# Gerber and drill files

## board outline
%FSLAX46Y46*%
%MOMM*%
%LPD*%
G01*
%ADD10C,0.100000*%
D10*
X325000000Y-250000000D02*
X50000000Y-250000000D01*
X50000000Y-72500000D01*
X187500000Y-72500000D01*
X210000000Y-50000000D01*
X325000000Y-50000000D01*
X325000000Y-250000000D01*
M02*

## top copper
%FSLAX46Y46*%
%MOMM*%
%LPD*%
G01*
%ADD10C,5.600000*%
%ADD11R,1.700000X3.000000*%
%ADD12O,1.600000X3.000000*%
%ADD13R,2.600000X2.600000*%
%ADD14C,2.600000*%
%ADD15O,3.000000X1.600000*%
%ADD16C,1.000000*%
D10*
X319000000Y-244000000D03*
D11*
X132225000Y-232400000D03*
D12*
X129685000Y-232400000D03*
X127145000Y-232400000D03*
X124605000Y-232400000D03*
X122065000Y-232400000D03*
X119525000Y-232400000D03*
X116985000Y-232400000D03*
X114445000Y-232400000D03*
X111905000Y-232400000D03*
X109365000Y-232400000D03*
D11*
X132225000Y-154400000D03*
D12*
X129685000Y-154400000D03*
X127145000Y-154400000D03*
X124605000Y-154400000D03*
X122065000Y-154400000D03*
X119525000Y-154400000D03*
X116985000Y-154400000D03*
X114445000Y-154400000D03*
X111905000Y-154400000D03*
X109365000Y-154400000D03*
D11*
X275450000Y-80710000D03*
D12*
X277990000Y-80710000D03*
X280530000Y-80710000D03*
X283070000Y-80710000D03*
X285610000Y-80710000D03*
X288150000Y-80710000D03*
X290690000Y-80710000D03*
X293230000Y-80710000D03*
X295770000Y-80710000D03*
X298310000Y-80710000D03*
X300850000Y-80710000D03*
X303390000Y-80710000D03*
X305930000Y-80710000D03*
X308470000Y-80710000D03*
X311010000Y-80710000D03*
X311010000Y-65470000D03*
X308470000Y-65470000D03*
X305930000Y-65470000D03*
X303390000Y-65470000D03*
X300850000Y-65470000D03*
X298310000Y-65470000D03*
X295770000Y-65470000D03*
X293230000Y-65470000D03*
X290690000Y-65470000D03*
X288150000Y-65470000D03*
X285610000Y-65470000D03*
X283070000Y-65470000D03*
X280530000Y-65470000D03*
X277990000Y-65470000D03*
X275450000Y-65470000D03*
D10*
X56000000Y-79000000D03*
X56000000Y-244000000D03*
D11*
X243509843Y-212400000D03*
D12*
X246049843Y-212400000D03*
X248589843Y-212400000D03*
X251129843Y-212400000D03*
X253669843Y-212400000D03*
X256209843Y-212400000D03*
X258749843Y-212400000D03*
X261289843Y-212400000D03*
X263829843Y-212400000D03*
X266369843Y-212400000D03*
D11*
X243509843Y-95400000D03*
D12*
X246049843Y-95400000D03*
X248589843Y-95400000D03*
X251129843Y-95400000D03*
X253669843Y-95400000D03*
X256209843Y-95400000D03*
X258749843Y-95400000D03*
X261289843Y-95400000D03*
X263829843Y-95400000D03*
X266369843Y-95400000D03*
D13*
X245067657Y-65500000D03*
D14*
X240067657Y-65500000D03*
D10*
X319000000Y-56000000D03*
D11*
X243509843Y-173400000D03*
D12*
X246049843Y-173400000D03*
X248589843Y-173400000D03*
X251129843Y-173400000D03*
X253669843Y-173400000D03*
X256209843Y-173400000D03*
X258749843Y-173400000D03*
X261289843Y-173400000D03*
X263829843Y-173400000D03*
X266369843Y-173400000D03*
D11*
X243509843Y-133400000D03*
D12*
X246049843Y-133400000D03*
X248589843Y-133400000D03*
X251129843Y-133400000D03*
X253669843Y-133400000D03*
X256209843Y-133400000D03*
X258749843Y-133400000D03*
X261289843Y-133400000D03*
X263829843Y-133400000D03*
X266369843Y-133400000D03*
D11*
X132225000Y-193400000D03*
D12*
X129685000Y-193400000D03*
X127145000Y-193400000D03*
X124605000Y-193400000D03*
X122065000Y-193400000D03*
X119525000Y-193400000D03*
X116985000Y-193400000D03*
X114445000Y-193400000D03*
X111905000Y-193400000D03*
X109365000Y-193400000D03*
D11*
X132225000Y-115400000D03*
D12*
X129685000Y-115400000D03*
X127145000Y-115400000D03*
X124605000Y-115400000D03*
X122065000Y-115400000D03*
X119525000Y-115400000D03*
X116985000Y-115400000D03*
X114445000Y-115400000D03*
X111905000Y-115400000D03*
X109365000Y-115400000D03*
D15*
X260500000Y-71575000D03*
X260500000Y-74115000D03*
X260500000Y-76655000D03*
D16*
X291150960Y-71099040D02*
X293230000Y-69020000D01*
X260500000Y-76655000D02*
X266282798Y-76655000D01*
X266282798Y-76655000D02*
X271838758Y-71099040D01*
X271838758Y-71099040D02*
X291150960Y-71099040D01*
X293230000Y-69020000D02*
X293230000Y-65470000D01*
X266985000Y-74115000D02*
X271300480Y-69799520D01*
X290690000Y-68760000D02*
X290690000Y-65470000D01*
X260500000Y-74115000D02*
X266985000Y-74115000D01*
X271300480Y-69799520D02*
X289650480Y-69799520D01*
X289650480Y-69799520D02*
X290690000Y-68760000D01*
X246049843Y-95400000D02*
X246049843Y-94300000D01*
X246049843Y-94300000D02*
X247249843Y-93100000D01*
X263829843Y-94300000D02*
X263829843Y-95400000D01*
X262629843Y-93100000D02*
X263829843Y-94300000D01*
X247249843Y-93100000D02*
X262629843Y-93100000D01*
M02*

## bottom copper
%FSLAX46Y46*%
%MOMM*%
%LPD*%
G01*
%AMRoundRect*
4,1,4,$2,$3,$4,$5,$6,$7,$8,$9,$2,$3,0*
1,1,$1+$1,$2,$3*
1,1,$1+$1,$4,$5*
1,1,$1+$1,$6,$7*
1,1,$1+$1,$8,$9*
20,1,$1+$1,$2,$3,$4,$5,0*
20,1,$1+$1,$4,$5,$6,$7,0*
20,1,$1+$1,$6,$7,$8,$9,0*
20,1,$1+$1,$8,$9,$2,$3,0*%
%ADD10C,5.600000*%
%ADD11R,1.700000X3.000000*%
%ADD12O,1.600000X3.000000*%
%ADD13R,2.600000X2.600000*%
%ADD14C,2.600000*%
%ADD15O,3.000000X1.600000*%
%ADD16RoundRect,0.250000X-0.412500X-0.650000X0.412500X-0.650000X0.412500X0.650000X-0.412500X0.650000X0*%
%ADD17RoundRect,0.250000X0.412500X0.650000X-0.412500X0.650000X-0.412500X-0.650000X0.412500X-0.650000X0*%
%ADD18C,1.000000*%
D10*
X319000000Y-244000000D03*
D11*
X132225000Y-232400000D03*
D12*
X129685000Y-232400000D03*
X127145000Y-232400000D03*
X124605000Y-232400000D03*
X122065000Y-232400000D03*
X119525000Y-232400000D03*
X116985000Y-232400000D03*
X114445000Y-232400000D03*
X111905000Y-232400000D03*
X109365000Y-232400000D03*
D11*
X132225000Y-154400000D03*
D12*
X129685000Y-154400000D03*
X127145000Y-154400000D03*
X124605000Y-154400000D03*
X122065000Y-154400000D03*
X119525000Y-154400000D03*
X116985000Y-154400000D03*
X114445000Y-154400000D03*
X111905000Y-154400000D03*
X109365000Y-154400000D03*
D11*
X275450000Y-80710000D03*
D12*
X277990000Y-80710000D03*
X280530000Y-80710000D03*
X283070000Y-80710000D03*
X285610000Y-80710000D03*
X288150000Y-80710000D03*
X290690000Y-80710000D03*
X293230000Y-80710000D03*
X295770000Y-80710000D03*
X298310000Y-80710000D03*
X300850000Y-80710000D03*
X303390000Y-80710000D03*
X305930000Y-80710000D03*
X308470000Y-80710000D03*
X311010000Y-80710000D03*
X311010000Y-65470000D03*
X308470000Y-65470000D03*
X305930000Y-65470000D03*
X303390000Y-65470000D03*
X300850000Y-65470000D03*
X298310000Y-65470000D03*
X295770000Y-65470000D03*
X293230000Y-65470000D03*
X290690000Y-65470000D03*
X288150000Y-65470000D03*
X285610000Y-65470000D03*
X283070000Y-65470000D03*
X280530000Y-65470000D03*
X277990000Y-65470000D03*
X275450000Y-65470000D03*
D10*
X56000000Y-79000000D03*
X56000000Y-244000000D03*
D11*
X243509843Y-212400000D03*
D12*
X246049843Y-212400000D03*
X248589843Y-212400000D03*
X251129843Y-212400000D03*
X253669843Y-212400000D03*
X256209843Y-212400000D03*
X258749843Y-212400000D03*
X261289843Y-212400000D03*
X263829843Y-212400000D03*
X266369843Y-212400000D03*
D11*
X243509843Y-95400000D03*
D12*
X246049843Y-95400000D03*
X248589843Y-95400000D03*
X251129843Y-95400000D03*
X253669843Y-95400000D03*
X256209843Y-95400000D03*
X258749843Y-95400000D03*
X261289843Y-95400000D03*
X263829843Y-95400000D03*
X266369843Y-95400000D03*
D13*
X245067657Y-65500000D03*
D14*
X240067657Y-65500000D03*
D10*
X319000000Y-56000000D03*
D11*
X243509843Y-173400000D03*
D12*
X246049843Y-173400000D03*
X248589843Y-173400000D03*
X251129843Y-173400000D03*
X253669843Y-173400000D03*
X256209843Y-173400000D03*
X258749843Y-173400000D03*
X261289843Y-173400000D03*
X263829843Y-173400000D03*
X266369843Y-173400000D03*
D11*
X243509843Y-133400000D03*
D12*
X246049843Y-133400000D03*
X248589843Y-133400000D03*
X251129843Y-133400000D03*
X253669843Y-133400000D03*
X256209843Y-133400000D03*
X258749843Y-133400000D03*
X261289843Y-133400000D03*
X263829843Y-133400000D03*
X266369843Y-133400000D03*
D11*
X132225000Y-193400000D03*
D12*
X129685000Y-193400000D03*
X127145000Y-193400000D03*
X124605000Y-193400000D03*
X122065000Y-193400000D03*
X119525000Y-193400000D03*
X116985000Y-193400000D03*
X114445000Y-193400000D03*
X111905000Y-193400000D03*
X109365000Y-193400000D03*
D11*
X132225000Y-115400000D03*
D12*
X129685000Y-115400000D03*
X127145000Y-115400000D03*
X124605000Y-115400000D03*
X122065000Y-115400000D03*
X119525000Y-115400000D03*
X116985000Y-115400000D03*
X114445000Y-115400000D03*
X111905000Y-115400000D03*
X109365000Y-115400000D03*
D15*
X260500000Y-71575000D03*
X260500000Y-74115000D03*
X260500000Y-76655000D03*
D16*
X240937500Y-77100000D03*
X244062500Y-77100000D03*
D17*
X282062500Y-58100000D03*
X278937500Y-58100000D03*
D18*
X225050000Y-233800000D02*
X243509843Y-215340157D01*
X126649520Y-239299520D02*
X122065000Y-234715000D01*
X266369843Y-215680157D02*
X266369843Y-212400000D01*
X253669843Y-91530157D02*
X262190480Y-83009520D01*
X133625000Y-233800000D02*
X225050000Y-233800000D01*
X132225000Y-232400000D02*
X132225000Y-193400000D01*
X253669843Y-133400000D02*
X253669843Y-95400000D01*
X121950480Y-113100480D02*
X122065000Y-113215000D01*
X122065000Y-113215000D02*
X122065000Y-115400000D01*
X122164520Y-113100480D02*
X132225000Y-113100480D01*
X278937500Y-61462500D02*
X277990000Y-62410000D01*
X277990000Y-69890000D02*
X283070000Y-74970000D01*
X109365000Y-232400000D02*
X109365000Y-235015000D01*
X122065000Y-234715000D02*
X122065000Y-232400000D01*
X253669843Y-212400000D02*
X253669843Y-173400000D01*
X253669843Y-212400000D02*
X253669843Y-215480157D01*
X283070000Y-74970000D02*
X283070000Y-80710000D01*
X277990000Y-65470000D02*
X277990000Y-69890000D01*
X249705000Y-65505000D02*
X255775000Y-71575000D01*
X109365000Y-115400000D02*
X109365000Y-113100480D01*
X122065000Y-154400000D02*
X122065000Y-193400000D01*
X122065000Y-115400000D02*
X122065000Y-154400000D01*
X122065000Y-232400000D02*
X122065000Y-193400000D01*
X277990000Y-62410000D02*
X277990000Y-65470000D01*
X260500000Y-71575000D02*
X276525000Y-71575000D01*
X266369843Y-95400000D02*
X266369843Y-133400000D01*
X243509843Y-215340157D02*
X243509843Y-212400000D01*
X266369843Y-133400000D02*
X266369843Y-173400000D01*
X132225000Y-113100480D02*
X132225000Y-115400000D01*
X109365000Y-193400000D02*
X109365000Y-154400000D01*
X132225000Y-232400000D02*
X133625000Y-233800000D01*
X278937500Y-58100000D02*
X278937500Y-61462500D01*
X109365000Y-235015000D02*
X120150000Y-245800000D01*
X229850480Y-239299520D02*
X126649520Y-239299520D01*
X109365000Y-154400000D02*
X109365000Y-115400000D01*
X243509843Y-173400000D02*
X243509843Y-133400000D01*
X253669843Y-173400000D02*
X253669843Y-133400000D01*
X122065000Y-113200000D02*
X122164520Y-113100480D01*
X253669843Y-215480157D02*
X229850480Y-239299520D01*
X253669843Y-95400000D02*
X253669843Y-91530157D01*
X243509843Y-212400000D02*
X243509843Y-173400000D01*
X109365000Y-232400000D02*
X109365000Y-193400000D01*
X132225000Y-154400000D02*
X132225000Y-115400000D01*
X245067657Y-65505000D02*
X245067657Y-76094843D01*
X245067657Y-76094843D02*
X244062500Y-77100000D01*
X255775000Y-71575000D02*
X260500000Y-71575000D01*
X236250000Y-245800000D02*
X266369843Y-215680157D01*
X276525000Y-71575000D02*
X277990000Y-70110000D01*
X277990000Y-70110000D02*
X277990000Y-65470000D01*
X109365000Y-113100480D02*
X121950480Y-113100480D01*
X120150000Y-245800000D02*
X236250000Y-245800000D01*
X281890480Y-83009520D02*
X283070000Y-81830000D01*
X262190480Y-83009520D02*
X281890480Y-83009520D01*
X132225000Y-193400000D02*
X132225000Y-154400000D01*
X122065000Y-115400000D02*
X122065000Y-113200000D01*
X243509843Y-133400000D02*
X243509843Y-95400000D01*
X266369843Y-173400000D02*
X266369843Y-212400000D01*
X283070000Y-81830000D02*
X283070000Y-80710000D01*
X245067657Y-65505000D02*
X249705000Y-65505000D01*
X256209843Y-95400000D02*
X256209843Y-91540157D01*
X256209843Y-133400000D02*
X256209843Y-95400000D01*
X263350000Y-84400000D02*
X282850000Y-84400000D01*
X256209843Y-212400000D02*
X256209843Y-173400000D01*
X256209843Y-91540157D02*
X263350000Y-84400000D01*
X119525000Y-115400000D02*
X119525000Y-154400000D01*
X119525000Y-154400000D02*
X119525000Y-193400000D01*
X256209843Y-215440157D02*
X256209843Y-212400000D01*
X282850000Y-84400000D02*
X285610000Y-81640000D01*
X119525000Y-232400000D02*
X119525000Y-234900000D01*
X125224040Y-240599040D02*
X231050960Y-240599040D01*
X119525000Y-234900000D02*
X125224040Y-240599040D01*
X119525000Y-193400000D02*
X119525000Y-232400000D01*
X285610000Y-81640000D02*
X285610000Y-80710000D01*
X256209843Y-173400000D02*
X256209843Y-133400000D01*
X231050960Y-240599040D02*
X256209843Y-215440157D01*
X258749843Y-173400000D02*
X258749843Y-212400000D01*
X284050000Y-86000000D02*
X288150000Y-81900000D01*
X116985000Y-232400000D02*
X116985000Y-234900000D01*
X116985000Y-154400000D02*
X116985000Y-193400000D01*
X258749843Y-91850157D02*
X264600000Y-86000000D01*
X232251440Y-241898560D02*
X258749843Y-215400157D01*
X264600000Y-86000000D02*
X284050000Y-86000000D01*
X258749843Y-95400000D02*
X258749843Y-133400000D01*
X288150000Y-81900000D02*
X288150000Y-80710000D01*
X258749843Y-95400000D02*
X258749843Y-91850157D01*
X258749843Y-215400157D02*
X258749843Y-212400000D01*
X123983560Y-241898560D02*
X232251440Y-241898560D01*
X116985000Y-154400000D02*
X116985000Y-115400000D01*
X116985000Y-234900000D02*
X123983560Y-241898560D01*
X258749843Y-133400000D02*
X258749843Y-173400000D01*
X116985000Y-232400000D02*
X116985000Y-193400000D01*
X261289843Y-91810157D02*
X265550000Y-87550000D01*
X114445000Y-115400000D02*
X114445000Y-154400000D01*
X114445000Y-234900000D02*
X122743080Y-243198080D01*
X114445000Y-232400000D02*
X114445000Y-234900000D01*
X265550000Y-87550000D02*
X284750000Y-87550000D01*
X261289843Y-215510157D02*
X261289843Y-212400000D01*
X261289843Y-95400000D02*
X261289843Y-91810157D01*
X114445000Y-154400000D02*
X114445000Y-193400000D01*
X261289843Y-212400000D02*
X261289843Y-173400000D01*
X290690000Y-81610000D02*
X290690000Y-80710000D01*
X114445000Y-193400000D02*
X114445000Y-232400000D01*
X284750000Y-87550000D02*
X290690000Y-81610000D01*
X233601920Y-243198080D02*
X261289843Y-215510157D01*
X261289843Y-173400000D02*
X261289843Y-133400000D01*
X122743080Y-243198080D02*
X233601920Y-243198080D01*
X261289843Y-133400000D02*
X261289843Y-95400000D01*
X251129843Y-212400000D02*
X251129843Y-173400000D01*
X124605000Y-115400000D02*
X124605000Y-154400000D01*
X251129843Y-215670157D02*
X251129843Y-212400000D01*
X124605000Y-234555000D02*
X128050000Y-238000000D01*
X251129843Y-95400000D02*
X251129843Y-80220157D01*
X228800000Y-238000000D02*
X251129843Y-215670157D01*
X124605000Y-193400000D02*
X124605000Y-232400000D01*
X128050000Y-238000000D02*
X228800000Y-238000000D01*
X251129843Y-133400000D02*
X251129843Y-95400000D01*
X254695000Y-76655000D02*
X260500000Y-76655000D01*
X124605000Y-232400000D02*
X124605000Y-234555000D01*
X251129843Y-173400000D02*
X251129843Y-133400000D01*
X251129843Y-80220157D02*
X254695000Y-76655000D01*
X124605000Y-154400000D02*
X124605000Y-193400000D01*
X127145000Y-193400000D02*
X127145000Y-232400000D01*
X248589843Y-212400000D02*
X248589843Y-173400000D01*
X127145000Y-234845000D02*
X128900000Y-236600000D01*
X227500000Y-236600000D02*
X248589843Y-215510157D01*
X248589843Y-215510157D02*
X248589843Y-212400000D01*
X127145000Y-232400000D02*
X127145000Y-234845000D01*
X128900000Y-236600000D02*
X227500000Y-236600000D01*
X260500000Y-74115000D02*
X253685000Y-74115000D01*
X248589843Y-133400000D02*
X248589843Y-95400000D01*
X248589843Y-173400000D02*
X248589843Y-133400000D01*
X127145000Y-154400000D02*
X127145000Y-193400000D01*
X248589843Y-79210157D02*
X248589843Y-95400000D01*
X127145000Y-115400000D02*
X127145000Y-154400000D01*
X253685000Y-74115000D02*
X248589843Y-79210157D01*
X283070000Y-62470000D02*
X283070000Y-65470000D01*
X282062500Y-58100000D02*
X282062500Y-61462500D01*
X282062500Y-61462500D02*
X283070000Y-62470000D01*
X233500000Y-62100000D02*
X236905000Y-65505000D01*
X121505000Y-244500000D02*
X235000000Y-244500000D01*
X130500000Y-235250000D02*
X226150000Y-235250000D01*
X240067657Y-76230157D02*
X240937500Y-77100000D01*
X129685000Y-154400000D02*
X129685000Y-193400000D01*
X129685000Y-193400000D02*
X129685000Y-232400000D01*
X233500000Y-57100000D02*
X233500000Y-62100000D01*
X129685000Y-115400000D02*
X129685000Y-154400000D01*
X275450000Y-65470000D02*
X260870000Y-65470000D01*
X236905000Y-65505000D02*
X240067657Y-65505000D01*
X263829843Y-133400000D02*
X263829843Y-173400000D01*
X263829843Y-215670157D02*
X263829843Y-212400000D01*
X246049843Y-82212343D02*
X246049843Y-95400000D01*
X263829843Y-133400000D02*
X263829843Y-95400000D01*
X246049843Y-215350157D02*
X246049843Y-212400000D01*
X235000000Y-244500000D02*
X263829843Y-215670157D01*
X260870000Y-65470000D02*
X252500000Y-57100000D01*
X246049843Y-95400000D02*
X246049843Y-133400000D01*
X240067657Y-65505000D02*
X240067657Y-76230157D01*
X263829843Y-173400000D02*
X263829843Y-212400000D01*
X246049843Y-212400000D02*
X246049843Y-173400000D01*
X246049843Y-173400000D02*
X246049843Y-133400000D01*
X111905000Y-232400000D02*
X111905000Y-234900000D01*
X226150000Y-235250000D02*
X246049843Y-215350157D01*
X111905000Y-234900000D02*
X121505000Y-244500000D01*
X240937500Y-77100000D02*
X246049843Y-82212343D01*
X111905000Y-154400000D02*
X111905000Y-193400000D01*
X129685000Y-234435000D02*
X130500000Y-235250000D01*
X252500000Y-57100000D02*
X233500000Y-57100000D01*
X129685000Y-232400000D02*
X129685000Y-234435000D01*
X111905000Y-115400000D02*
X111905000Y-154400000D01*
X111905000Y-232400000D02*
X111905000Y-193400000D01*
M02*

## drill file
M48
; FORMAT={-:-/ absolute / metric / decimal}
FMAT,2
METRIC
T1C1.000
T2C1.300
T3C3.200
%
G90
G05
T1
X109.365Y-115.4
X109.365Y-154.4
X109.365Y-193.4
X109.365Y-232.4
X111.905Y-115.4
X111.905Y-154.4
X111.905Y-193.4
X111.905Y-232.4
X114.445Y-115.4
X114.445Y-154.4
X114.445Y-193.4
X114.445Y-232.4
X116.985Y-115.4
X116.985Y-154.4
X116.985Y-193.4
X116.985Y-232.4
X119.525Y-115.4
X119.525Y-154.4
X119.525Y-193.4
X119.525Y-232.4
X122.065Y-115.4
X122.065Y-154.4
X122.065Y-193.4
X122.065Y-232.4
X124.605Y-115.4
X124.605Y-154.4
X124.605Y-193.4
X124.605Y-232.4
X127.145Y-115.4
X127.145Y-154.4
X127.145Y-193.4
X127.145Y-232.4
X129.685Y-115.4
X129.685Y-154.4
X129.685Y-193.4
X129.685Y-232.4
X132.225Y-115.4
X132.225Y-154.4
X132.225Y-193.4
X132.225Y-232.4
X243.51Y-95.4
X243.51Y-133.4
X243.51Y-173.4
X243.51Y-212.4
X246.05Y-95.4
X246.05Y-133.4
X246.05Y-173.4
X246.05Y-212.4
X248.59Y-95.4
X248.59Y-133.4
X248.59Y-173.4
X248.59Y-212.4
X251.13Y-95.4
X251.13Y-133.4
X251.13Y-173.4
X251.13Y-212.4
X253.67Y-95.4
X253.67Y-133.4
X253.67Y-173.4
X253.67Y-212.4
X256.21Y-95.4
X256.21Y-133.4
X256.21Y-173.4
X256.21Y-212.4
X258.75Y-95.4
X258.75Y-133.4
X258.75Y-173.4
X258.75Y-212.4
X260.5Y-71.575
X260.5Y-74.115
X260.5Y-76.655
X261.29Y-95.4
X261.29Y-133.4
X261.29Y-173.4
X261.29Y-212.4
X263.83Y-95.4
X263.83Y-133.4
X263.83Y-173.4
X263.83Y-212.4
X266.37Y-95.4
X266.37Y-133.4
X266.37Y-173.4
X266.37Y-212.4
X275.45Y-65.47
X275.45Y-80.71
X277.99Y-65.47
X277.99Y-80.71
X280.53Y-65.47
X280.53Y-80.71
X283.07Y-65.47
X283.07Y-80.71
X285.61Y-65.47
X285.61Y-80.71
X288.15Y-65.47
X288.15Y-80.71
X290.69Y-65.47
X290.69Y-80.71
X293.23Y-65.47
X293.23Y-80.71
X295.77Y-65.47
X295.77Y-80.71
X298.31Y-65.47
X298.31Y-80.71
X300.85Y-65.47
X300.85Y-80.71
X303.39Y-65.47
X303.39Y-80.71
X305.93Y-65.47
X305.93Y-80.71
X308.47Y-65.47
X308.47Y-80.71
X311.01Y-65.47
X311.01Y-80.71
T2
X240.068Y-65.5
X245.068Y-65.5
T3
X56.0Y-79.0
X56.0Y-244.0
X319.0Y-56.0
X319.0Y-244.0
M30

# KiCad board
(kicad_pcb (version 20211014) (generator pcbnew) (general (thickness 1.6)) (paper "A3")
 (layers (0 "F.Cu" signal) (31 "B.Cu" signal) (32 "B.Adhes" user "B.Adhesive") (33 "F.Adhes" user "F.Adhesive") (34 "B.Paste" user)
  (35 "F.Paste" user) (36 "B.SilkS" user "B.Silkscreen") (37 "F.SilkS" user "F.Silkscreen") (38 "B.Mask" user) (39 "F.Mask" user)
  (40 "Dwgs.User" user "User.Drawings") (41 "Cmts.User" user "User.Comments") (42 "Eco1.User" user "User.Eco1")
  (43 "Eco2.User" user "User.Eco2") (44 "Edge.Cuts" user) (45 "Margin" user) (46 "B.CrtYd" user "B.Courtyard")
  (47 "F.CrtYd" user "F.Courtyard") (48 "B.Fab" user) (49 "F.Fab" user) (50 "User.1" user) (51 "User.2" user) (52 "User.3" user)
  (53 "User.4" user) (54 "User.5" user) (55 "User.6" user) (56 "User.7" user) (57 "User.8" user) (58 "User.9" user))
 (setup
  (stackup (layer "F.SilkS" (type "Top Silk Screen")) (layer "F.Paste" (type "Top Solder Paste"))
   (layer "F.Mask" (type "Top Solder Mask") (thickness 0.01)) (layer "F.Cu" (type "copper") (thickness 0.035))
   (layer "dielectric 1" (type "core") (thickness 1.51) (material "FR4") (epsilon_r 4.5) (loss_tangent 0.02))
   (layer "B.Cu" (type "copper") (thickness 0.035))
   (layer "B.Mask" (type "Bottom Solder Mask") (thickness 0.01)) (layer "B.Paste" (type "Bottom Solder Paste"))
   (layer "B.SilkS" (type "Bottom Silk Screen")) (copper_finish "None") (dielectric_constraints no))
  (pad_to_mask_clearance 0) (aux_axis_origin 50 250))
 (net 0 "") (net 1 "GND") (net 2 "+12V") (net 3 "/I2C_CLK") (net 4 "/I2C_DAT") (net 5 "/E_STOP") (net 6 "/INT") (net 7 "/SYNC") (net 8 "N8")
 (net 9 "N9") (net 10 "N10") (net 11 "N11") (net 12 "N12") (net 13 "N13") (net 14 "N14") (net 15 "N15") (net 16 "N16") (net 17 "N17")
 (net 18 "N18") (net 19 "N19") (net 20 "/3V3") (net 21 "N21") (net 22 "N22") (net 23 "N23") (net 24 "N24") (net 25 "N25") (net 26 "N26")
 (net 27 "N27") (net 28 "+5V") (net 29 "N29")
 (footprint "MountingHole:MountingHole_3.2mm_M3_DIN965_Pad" (layer "F.Cu") (at 319 244)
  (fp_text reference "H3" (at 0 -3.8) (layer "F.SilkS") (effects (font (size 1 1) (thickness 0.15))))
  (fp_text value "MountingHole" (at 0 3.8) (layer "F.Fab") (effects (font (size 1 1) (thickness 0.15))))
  (pad "1" thru_hole circle (at 0 0) (size 5.6 5.6) (drill 3.2) (layers *.Cu *.Mask)))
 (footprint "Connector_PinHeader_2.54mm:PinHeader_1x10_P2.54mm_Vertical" (layer "F.Cu") (at 132.225 232.4 -90)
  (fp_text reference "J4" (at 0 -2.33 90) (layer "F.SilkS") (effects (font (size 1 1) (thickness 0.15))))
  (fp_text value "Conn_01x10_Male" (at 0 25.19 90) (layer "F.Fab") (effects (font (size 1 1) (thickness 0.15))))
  (pad "1" thru_hole rect (at 0 0) (size 1.7 3) (drill 1) (layers *.Cu *.Mask) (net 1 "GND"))
  (pad "2" thru_hole oval (at 0 2.54) (size 1.6 3) (drill 1) (layers *.Cu *.Mask) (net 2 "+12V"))
  (pad "3" thru_hole oval (at 0 5.08) (size 1.6 3) (drill 1) (layers *.Cu *.Mask) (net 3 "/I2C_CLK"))
  (pad "4" thru_hole oval (at 0 7.62) (size 1.6 3) (drill 1) (layers *.Cu *.Mask) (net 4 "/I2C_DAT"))
  (pad "5" thru_hole oval (at 0 10.16) (size 1.6 3) (drill 1) (layers *.Cu *.Mask) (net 1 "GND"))
  (pad "6" thru_hole oval (at 0 12.7) (size 1.6 3) (drill 1) (layers *.Cu *.Mask) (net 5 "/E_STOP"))
  (pad "7" thru_hole oval (at 0 15.24) (size 1.6 3) (drill 1) (layers *.Cu *.Mask) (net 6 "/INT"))
  (pad "8" thru_hole oval (at 0 17.78) (size 1.6 3) (drill 1) (layers *.Cu *.Mask) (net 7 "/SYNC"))
  (pad "9" thru_hole oval (at 0 20.32) (size 1.6 3) (drill 1) (layers *.Cu *.Mask) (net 2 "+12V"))
  (pad "10" thru_hole oval (at 0 22.86) (size 1.6 3) (drill 1) (layers *.Cu *.Mask) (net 1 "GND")))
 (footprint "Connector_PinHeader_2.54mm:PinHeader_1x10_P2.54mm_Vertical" (layer "F.Cu") (at 132.225 154.4 -90)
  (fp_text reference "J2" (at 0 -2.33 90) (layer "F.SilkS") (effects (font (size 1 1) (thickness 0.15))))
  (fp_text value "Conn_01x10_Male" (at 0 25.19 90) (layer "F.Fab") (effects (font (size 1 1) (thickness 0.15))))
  (pad "1" thru_hole rect (at 0 0) (size 1.7 3) (drill 1) (layers *.Cu *.Mask) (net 1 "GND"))
  (pad "2" thru_hole oval (at 0 2.54) (size 1.6 3) (drill 1) (layers *.Cu *.Mask) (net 2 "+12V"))
  (pad "3" thru_hole oval (at 0 5.08) (size 1.6 3) (drill 1) (layers *.Cu *.Mask) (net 3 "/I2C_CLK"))
  (pad "4" thru_hole oval (at 0 7.62) (size 1.6 3) (drill 1) (layers *.Cu *.Mask) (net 4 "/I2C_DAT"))
  (pad "5" thru_hole oval (at 0 10.16) (size 1.6 3) (drill 1) (layers *.Cu *.Mask) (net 1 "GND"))
  (pad "6" thru_hole oval (at 0 12.7) (size 1.6 3) (drill 1) (layers *.Cu *.Mask) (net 5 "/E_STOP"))
  (pad "7" thru_hole oval (at 0 15.24) (size 1.6 3) (drill 1) (layers *.Cu *.Mask) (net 6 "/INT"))
  (pad "8" thru_hole oval (at 0 17.78) (size 1.6 3) (drill 1) (layers *.Cu *.Mask) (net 7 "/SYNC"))
  (pad "9" thru_hole oval (at 0 20.32) (size 1.6 3) (drill 1) (layers *.Cu *.Mask) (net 2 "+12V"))
  (pad "10" thru_hole oval (at 0 22.86) (size 1.6 3) (drill 1) (layers *.Cu *.Mask) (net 1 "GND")))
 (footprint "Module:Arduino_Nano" (layer "F.Cu") (at 275.45 80.71 90)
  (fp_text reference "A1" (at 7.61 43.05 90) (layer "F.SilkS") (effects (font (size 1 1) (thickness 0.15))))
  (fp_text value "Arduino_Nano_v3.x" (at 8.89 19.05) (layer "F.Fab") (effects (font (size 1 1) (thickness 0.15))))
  (pad "1" thru_hole rect (at 0 0 180) (size 1.7 3) (drill 1) (layers *.Cu *.Mask) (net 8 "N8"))
  (pad "2" thru_hole oval (at 0 2.54 180) (size 1.6 3) (drill 1) (layers *.Cu *.Mask) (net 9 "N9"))
  (pad "3" thru_hole oval (at 0 5.08 180) (size 1.6 3) (drill 1) (layers *.Cu *.Mask) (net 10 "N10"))
  (pad "4" thru_hole oval (at 0 7.62 180) (size 1.6 3) (drill 1) (layers *.Cu *.Mask) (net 1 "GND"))
  (pad "5" thru_hole oval (at 0 10.16 180) (size 1.6 3) (drill 1) (layers *.Cu *.Mask) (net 5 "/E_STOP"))
  (pad "6" thru_hole oval (at 0 12.7 180) (size 1.6 3) (drill 1) (layers *.Cu *.Mask) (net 6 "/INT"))
  (pad "7" thru_hole oval (at 0 15.24 180) (size 1.6 3) (drill 1) (layers *.Cu *.Mask) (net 7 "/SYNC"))
  (pad "8" thru_hole oval (at 0 17.78 180) (size 1.6 3) (drill 1) (layers *.Cu *.Mask) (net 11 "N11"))
  (pad "9" thru_hole oval (at 0 20.32 180) (size 1.6 3) (drill 1) (layers *.Cu *.Mask) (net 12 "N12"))
  (pad "10" thru_hole oval (at 0 22.86 180) (size 1.6 3) (drill 1) (layers *.Cu *.Mask) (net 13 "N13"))
  (pad "11" thru_hole oval (at 0 25.4 180) (size 1.6 3) (drill 1) (layers *.Cu *.Mask) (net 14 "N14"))
  (pad "12" thru_hole oval (at 0 27.94 180) (size 1.6 3) (drill 1) (layers *.Cu *.Mask) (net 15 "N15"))
  (pad "13" thru_hole oval (at 0 30.48 180) (size 1.6 3) (drill 1) (layers *.Cu *.Mask) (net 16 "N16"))
  (pad "14" thru_hole oval (at 0 33.02 180) (size 1.6 3) (drill 1) (layers *.Cu *.Mask) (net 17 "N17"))
  (pad "15" thru_hole oval (at 0 35.56 180) (size 1.6 3) (drill 1) (layers *.Cu *.Mask) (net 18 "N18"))
  (pad "16" thru_hole oval (at 15.24 35.56 180) (size 1.6 3) (drill 1) (layers *.Cu *.Mask) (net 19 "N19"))
  (pad "17" thru_hole oval (at 15.24 33.02 180) (size 1.6 3) (drill 1) (layers *.Cu *.Mask) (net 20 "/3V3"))
  (pad "18" thru_hole oval (at 15.24 30.48 180) (size 1.6 3) (drill 1) (layers *.Cu *.Mask) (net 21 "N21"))
  (pad "19" thru_hole oval (at 15.24 27.94 180) (size 1.6 3) (drill 1) (layers *.Cu *.Mask) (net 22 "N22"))
  (pad "20" thru_hole oval (at 15.24 25.4 180) (size 1.6 3) (drill 1) (layers *.Cu *.Mask) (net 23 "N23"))
  (pad "21" thru_hole oval (at 15.24 22.86 180) (size 1.6 3) (drill 1) (layers *.Cu *.Mask) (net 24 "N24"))
  (pad "22" thru_hole oval (at 15.24 20.32 180) (size 1.6 3) (drill 1) (layers *.Cu *.Mask) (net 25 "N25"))
  (pad "23" thru_hole oval (at 15.24 17.78 180) (size 1.6 3) (drill 1) (layers *.Cu *.Mask) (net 4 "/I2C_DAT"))
  (pad "24" thru_hole oval (at 15.24 15.24 180) (size 1.6 3) (drill 1) (layers *.Cu *.Mask) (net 3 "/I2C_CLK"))
  (pad "25" thru_hole oval (at 15.24 12.7 180) (size 1.6 3) (drill 1) (layers *.Cu *.Mask) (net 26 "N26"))
  (pad "26" thru_hole oval (at 15.24 10.16 180) (size 1.6 3) (drill 1) (layers *.Cu *.Mask) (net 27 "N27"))
  (pad "27" thru_hole oval (at 15.24 7.62 180) (size 1.6 3) (drill 1) (layers *.Cu *.Mask) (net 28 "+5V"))
  (pad "28" thru_hole oval (at 15.24 5.08 180) (size 1.6 3) (drill 1) (layers *.Cu *.Mask) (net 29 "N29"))
  (pad "29" thru_hole oval (at 15.24 2.54 180) (size 1.6 3) (drill 1) (layers *.Cu *.Mask) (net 1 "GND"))
  (pad "30" thru_hole oval (at 15.24 0 180) (size 1.6 3) (drill 1) (layers *.Cu *.Mask) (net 2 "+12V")))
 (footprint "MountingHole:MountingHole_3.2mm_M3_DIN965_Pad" (layer "F.Cu") (at 56 79)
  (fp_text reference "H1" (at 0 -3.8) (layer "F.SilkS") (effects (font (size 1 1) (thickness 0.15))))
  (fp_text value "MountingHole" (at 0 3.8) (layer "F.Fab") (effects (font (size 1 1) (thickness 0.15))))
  (pad "1" thru_hole circle (at 0 0) (size 5.6 5.6) (drill 3.2) (layers *.Cu *.Mask)))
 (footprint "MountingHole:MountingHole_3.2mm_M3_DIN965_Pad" (layer "F.Cu") (at 56 244)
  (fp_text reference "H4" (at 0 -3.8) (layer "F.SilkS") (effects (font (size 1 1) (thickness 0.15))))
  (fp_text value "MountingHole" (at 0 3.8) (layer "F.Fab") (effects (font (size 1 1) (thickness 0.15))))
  (pad "1" thru_hole circle (at 0 0) (size 5.6 5.6) (drill 3.2) (layers *.Cu *.Mask)))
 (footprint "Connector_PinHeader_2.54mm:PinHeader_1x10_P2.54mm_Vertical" (layer "F.Cu") (at 243.509843 212.4 90)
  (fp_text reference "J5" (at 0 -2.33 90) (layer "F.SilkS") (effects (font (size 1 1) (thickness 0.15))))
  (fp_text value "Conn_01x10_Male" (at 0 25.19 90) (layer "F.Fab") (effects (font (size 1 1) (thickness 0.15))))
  (pad "1" thru_hole rect (at 0 0 180) (size 1.7 3) (drill 1) (layers *.Cu *.Mask) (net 1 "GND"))
  (pad "2" thru_hole oval (at 0 2.54 180) (size 1.6 3) (drill 1) (layers *.Cu *.Mask) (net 2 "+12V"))
  (pad "3" thru_hole oval (at 0 5.08 180) (size 1.6 3) (drill 1) (layers *.Cu *.Mask) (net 3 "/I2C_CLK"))
  (pad "4" thru_hole oval (at 0 7.62 180) (size 1.6 3) (drill 1) (layers *.Cu *.Mask) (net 4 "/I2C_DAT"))
  (pad "5" thru_hole oval (at 0 10.16 180) (size 1.6 3) (drill 1) (layers *.Cu *.Mask) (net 1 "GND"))
  (pad "6" thru_hole oval (at 0 12.7 180) (size 1.6 3) (drill 1) (layers *.Cu *.Mask) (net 5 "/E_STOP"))
  (pad "7" thru_hole oval (at 0 15.24 180) (size 1.6 3) (drill 1) (layers *.Cu *.Mask) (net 6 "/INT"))
  (pad "8" thru_hole oval (at 0 17.78 180) (size 1.6 3) (drill 1) (layers *.Cu *.Mask) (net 7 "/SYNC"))
  (pad "9" thru_hole oval (at 0 20.32 180) (size 1.6 3) (drill 1) (layers *.Cu *.Mask) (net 2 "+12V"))
  (pad "10" thru_hole oval (at 0 22.86 180) (size 1.6 3) (drill 1) (layers *.Cu *.Mask) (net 1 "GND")))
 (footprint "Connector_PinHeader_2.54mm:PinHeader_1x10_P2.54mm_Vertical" (layer "F.Cu") (at 243.509843 95.4 90)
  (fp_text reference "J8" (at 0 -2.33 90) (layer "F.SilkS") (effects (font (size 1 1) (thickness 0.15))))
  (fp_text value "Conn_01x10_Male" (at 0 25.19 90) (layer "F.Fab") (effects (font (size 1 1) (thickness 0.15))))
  (pad "1" thru_hole rect (at 0 0 180) (size 1.7 3) (drill 1) (layers *.Cu *.Mask) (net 1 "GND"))
  (pad "2" thru_hole oval (at 0 2.54 180) (size 1.6 3) (drill 1) (layers *.Cu *.Mask) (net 2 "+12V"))
  (pad "3" thru_hole oval (at 0 5.08 180) (size 1.6 3) (drill 1) (layers *.Cu *.Mask) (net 3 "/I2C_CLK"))
  (pad "4" thru_hole oval (at 0 7.62 180) (size 1.6 3) (drill 1) (layers *.Cu *.Mask) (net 4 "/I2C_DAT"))
  (pad "5" thru_hole oval (at 0 10.16 180) (size 1.6 3) (drill 1) (layers *.Cu *.Mask) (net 1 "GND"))
  (pad "6" thru_hole oval (at 0 12.7 180) (size 1.6 3) (drill 1) (layers *.Cu *.Mask) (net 5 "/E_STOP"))
  (pad "7" thru_hole oval (at 0 15.24 180) (size 1.6 3) (drill 1) (layers *.Cu *.Mask) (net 6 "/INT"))
  (pad "8" thru_hole oval (at 0 17.78 180) (size 1.6 3) (drill 1) (layers *.Cu *.Mask) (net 7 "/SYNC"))
  (pad "9" thru_hole oval (at 0 20.32 180) (size 1.6 3) (drill 1) (layers *.Cu *.Mask) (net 2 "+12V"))
  (pad "10" thru_hole oval (at 0 22.86 180) (size 1.6 3) (drill 1) (layers *.Cu *.Mask) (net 1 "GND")))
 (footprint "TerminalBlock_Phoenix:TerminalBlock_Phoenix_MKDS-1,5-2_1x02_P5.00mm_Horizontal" (layer "F.Cu") (at 245.067657 65.5 180)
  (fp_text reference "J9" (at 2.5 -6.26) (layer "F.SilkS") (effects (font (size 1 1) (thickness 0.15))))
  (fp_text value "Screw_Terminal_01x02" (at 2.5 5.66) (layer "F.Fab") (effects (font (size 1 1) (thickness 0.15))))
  (pad "1" thru_hole rect (at 0 0 180) (size 2.6 2.6) (drill 1.3) (layers *.Cu *.Mask) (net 1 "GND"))
  (pad "2" thru_hole circle (at 5 0 180) (size 2.6 2.6) (drill 1.3) (layers *.Cu *.Mask) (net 2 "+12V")))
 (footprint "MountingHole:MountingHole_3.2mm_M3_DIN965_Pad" (layer "F.Cu") (at 319 56)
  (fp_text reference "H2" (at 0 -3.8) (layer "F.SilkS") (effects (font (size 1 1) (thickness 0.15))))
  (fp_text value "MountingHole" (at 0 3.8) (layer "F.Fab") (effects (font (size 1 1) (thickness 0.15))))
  (pad "1" thru_hole circle (at 0 0) (size 5.6 5.6) (drill 3.2) (layers *.Cu *.Mask)))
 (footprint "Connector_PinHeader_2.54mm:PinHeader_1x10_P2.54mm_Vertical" (layer "F.Cu") (at 243.509843 173.4 90)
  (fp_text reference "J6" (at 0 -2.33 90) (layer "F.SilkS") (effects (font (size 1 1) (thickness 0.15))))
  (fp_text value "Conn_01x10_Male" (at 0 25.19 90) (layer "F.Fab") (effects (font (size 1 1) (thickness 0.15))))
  (pad "1" thru_hole rect (at 0 0 180) (size 1.7 3) (drill 1) (layers *.Cu *.Mask) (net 1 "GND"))
  (pad "2" thru_hole oval (at 0 2.54 180) (size 1.6 3) (drill 1) (layers *.Cu *.Mask) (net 2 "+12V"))
  (pad "3" thru_hole oval (at 0 5.08 180) (size 1.6 3) (drill 1) (layers *.Cu *.Mask) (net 3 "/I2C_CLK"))
  (pad "4" thru_hole oval (at 0 7.62 180) (size 1.6 3) (drill 1) (layers *.Cu *.Mask) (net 4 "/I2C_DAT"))
  (pad "5" thru_hole oval (at 0 10.16 180) (size 1.6 3) (drill 1) (layers *.Cu *.Mask) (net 1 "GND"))
  (pad "6" thru_hole oval (at 0 12.7 180) (size 1.6 3) (drill 1) (layers *.Cu *.Mask) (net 5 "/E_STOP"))
  (pad "7" thru_hole oval (at 0 15.24 180) (size 1.6 3) (drill 1) (layers *.Cu *.Mask) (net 6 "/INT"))
  (pad "8" thru_hole oval (at 0 17.78 180) (size 1.6 3) (drill 1) (layers *.Cu *.Mask) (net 7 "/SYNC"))
  (pad "9" thru_hole oval (at 0 20.32 180) (size 1.6 3) (drill 1) (layers *.Cu *.Mask) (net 2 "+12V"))
  (pad "10" thru_hole oval (at 0 22.86 180) (size 1.6 3) (drill 1) (layers *.Cu *.Mask) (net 1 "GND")))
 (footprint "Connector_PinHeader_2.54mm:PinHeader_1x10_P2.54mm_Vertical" (layer "F.Cu") (at 243.509843 133.4 90)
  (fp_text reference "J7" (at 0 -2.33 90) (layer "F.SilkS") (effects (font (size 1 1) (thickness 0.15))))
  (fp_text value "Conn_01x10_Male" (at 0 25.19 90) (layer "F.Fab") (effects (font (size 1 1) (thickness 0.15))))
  (pad "1" thru_hole rect (at 0 0 180) (size 1.7 3) (drill 1) (layers *.Cu *.Mask) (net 1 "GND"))
  (pad "2" thru_hole oval (at 0 2.54 180) (size 1.6 3) (drill 1) (layers *.Cu *.Mask) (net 2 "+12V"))
  (pad "3" thru_hole oval (at 0 5.08 180) (size 1.6 3) (drill 1) (layers *.Cu *.Mask) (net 3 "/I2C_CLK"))
  (pad "4" thru_hole oval (at 0 7.62 180) (size 1.6 3) (drill 1) (layers *.Cu *.Mask) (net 4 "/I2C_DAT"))
  (pad "5" thru_hole oval (at 0 10.16 180) (size 1.6 3) (drill 1) (layers *.Cu *.Mask) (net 1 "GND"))
  (pad "6" thru_hole oval (at 0 12.7 180) (size 1.6 3) (drill 1) (layers *.Cu *.Mask) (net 5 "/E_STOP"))
  (pad "7" thru_hole oval (at 0 15.24 180) (size 1.6 3) (drill 1) (layers *.Cu *.Mask) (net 6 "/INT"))
  (pad "8" thru_hole oval (at 0 17.78 180) (size 1.6 3) (drill 1) (layers *.Cu *.Mask) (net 7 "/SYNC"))
  (pad "9" thru_hole oval (at 0 20.32 180) (size 1.6 3) (drill 1) (layers *.Cu *.Mask) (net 2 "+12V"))
  (pad "10" thru_hole oval (at 0 22.86 180) (size 1.6 3) (drill 1) (layers *.Cu *.Mask) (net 1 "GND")))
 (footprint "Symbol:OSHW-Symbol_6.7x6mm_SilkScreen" (layer "F.Cu") (at 306.5 244.5)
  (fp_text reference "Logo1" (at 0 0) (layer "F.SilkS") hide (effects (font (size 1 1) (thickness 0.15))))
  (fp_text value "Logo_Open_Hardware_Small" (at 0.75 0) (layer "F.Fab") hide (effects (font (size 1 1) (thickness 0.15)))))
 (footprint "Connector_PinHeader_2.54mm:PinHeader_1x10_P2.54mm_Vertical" (layer "F.Cu") (at 132.225 193.4 -90)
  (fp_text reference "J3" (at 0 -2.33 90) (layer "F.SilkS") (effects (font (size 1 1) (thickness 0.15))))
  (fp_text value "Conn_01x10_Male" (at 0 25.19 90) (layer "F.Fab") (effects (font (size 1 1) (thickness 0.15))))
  (pad "1" thru_hole rect (at 0 0) (size 1.7 3) (drill 1) (layers *.Cu *.Mask) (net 1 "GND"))
  (pad "2" thru_hole oval (at 0 2.54) (size 1.6 3) (drill 1) (layers *.Cu *.Mask) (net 2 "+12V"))
  (pad "3" thru_hole oval (at 0 5.08) (size 1.6 3) (drill 1) (layers *.Cu *.Mask) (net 3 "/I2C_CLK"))
  (pad "4" thru_hole oval (at 0 7.62) (size 1.6 3) (drill 1) (layers *.Cu *.Mask) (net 4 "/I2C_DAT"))
  (pad "5" thru_hole oval (at 0 10.16) (size 1.6 3) (drill 1) (layers *.Cu *.Mask) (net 1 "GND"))
  (pad "6" thru_hole oval (at 0 12.7) (size 1.6 3) (drill 1) (layers *.Cu *.Mask) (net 5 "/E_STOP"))
  (pad "7" thru_hole oval (at 0 15.24) (size 1.6 3) (drill 1) (layers *.Cu *.Mask) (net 6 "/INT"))
  (pad "8" thru_hole oval (at 0 17.78) (size 1.6 3) (drill 1) (layers *.Cu *.Mask) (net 7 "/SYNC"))
  (pad "9" thru_hole oval (at 0 20.32) (size 1.6 3) (drill 1) (layers *.Cu *.Mask) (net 2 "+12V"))
  (pad "10" thru_hole oval (at 0 22.86) (size 1.6 3) (drill 1) (layers *.Cu *.Mask) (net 1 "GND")))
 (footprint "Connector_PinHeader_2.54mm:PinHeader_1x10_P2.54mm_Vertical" (layer "F.Cu") (at 132.225 115.4 -90)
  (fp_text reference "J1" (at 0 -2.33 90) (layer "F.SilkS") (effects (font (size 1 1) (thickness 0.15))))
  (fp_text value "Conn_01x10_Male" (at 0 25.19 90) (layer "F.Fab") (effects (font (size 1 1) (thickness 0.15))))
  (pad "1" thru_hole rect (at 0 0) (size 1.7 3) (drill 1) (layers *.Cu *.Mask) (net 1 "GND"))
  (pad "2" thru_hole oval (at 0 2.54) (size 1.6 3) (drill 1) (layers *.Cu *.Mask) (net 2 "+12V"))
  (pad "3" thru_hole oval (at 0 5.08) (size 1.6 3) (drill 1) (layers *.Cu *.Mask) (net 3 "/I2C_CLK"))
  (pad "4" thru_hole oval (at 0 7.62) (size 1.6 3) (drill 1) (layers *.Cu *.Mask) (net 4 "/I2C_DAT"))
  (pad "5" thru_hole oval (at 0 10.16) (size 1.6 3) (drill 1) (layers *.Cu *.Mask) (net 1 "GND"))
  (pad "6" thru_hole oval (at 0 12.7) (size 1.6 3) (drill 1) (layers *.Cu *.Mask) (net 5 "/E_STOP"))
  (pad "7" thru_hole oval (at 0 15.24) (size 1.6 3) (drill 1) (layers *.Cu *.Mask) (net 6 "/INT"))
  (pad "8" thru_hole oval (at 0 17.78) (size 1.6 3) (drill 1) (layers *.Cu *.Mask) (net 7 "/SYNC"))
  (pad "9" thru_hole oval (at 0 20.32) (size 1.6 3) (drill 1) (layers *.Cu *.Mask) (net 2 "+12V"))
  (pad "10" thru_hole oval (at 0 22.86) (size 1.6 3) (drill 1) (layers *.Cu *.Mask) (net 1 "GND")))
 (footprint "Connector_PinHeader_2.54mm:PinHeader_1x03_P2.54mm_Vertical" (layer "F.Cu") (at 260.5 71.575)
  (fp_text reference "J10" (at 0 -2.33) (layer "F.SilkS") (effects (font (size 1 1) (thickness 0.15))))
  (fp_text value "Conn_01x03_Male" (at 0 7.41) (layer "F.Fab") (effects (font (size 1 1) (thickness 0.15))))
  (pad "1" thru_hole oval (at 0 0 90) (size 1.6 3) (drill 1) (layers *.Cu *.Mask) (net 1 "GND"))
  (pad "2" thru_hole oval (at 0 2.54 90) (size 1.6 3) (drill 1) (layers *.Cu *.Mask) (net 3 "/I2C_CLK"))
  (pad "3" thru_hole oval (at 0 5.08 90) (size 1.6 3) (drill 1) (layers *.Cu *.Mask) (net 4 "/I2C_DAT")))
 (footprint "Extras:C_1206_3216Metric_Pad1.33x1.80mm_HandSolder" (layer "B.Cu") (at 242.5 77.1)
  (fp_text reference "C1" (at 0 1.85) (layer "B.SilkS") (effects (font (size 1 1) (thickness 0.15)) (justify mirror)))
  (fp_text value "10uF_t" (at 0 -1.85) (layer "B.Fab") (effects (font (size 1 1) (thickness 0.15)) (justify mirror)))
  (pad "1" smd roundrect (at -1.5625 0) (size 1.325 1.8) (layers "B.Cu" "B.Paste" "B.Mask") (roundrect_rratio 0.1886792453) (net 2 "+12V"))
  (pad "2" smd roundrect (at 1.5625 0) (size 1.325 1.8) (layers "B.Cu" "B.Paste" "B.Mask") (roundrect_rratio 0.1886792453) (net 1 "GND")))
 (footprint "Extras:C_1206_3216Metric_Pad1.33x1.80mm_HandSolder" (layer "B.Cu") (at 280.5 58.1 180)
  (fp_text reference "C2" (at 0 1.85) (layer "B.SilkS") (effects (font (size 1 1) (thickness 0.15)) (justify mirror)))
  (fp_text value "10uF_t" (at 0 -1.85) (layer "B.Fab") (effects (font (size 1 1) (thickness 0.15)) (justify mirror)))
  (pad "1" smd roundrect (at -1.5625 0 180) (size 1.325 1.8) (layers "B.Cu" "B.Paste" "B.Mask") (roundrect_rratio 0.1886792453)
   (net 28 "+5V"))
  (pad "2" smd roundrect (at 1.5625 0 180) (size 1.325 1.8) (layers "B.Cu" "B.Paste" "B.Mask") (roundrect_rratio 0.1886792453) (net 1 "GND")))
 (gr_poly (pts (xy 325 250) (xy 50 250) (xy 50 72.5) (xy 187.5 72.5) (xy 210 50) (xy 325 50)) (layer "Edge.Cuts") (width 0.1) (fill none))
 (segment (start 225.05 233.8) (end 243.509843 215.340157) (width 1) (layer "B.Cu") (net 1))
 (segment (start 126.64952 239.29952) (end 122.065 234.715) (width 1) (layer "B.Cu") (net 1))
 (segment (start 266.369843 215.680157) (end 266.369843 212.4) (width 1) (layer "B.Cu") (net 1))
 (segment (start 253.669843 91.530157) (end 262.19048 83.00952) (width 1) (layer "B.Cu") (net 1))
 (segment (start 133.625 233.8) (end 225.05 233.8) (width 1) (layer "B.Cu") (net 1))
 (segment (start 132.225 232.4) (end 132.225 193.4) (width 1) (layer "B.Cu") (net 1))
 (segment (start 253.669843 133.4) (end 253.669843 95.4) (width 1) (layer "B.Cu") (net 1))
 (segment (start 121.95048 113.10048) (end 122.065 113.215) (width 1) (layer "B.Cu") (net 1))
 (segment (start 122.065 113.215) (end 122.065 115.4) (width 1) (layer "B.Cu") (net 1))
 (segment (start 122.16452 113.10048) (end 132.225 113.10048) (width 1) (layer "B.Cu") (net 1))
 (segment (start 278.9375 61.4625) (end 277.99 62.41) (width 1) (layer "B.Cu") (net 1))
 (segment (start 277.99 69.89) (end 283.07 74.97) (width 1) (layer "B.Cu") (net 1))
 (segment (start 109.365 232.4) (end 109.365 235.015) (width 1) (layer "B.Cu") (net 1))
 (segment (start 122.065 234.715) (end 122.065 232.4) (width 1) (layer "B.Cu") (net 1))
 (segment (start 253.669843 212.4) (end 253.669843 173.4) (width 1) (layer "B.Cu") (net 1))
 (segment (start 253.669843 212.4) (end 253.669843 215.480157) (width 1) (layer "B.Cu") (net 1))
 (segment (start 283.07 74.97) (end 283.07 80.71) (width 1) (layer "B.Cu") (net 1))
 (segment (start 277.99 65.47) (end 277.99 69.89) (width 1) (layer "B.Cu") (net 1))
 (segment (start 249.705 65.505) (end 255.775 71.575) (width 1) (layer "B.Cu") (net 1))
 (segment (start 109.365 115.4) (end 109.365 113.10048) (width 1) (layer "B.Cu") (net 1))
 (segment (start 122.065 154.4) (end 122.065 193.4) (width 1) (layer "B.Cu") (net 1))
 (segment (start 122.065 115.4) (end 122.065 154.4) (width 1) (layer "B.Cu") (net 1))
 (segment (start 122.065 232.4) (end 122.065 193.4) (width 1) (layer "B.Cu") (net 1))
 (segment (start 277.99 62.41) (end 277.99 65.47) (width 1) (layer "B.Cu") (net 1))
 (segment (start 260.5 71.575) (end 276.525 71.575) (width 1) (layer "B.Cu") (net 1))
 (segment (start 266.369843 95.4) (end 266.369843 133.4) (width 1) (layer "B.Cu") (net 1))
 (segment (start 243.509843 215.340157) (end 243.509843 212.4) (width 1) (layer "B.Cu") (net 1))
 (segment (start 266.369843 133.4) (end 266.369843 173.4) (width 1) (layer "B.Cu") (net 1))
 (segment (start 132.225 113.10048) (end 132.225 115.4) (width 1) (layer "B.Cu") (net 1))
 (segment (start 109.365 193.4) (end 109.365 154.4) (width 1) (layer "B.Cu") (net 1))
 (segment (start 132.225 232.4) (end 133.625 233.8) (width 1) (layer "B.Cu") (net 1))
 (segment (start 278.9375 58.1) (end 278.9375 61.4625) (width 1) (layer "B.Cu") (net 1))
 (segment (start 109.365 235.015) (end 120.15 245.8) (width 1) (layer "B.Cu") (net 1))
 (segment (start 229.85048 239.29952) (end 126.64952 239.29952) (width 1) (layer "B.Cu") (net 1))
 (segment (start 109.365 154.4) (end 109.365 115.4) (width 1) (layer "B.Cu") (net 1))
 (segment (start 243.509843 173.4) (end 243.509843 133.4) (width 1) (layer "B.Cu") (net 1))
 (segment (start 253.669843 173.4) (end 253.669843 133.4) (width 1) (layer "B.Cu") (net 1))
 (segment (start 122.065 113.2) (end 122.16452 113.10048) (width 1) (layer "B.Cu") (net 1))
 (segment (start 253.669843 215.480157) (end 229.85048 239.29952) (width 1) (layer "B.Cu") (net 1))
 (segment (start 253.669843 95.4) (end 253.669843 91.530157) (width 1) (layer "B.Cu") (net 1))
 (segment (start 243.509843 212.4) (end 243.509843 173.4) (width 1) (layer "B.Cu") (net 1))
 (segment (start 109.365 232.4) (end 109.365 193.4) (width 1) (layer "B.Cu") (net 1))
 (segment (start 132.225 154.4) (end 132.225 115.4) (width 1) (layer "B.Cu") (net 1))
 (segment (start 245.067657 65.505) (end 245.067657 76.094843) (width 1) (layer "B.Cu") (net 1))
 (segment (start 245.067657 76.094843) (end 244.0625 77.1) (width 1) (layer "B.Cu") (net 1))
 (segment (start 255.775 71.575) (end 260.5 71.575) (width 1) (layer "B.Cu") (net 1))
 (segment (start 236.25 245.8) (end 266.369843 215.680157) (width 1) (layer "B.Cu") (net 1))
 (segment (start 276.525 71.575) (end 277.99 70.11) (width 1) (layer "B.Cu") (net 1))
 (segment (start 277.99 70.11) (end 277.99 65.47) (width 1) (layer "B.Cu") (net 1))
 (segment (start 109.365 113.10048) (end 121.95048 113.10048) (width 1) (layer "B.Cu") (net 1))
 (segment (start 120.15 245.8) (end 236.25 245.8) (width 1) (layer "B.Cu") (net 1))
 (segment (start 281.89048 83.00952) (end 283.07 81.83) (width 1) (layer "B.Cu") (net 1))
 (segment (start 262.19048 83.00952) (end 281.89048 83.00952) (width 1) (layer "B.Cu") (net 1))
 (segment (start 132.225 193.4) (end 132.225 154.4) (width 1) (layer "B.Cu") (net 1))
 (segment (start 122.065 115.4) (end 122.065 113.2) (width 1) (layer "B.Cu") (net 1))
 (segment (start 243.509843 133.4) (end 243.509843 95.4) (width 1) (layer "B.Cu") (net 1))
 (segment (start 266.369843 173.4) (end 266.369843 212.4) (width 1) (layer "B.Cu") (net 1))
 (segment (start 283.07 81.83) (end 283.07 80.71) (width 1) (layer "B.Cu") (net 1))
 (segment (start 245.067657 65.505) (end 249.705 65.505) (width 1) (layer "B.Cu") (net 1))
 (segment (start 256.209843 95.4) (end 256.209843 91.540157) (width 1) (layer "B.Cu") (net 5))
 (segment (start 256.209843 133.4) (end 256.209843 95.4) (width 1) (layer "B.Cu") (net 5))
 (segment (start 263.35 84.4) (end 282.85 84.4) (width 1) (layer "B.Cu") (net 5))
 (segment (start 256.209843 212.4) (end 256.209843 173.4) (width 1) (layer "B.Cu") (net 5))
 (segment (start 256.209843 91.540157) (end 263.35 84.4) (width 1) (layer "B.Cu") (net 5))
 (segment (start 119.525 115.4) (end 119.525 154.4) (width 1) (layer "B.Cu") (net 5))
 (segment (start 119.525 154.4) (end 119.525 193.4) (width 1) (layer "B.Cu") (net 5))
 (segment (start 256.209843 215.440157) (end 256.209843 212.4) (width 1) (layer "B.Cu") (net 5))
 (segment (start 282.85 84.4) (end 285.61 81.64) (width 1) (layer "B.Cu") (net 5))
 (segment (start 119.525 232.4) (end 119.525 234.9) (width 1) (layer "B.Cu") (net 5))
 (segment (start 125.22404 240.59904) (end 231.05096 240.59904) (width 1) (layer "B.Cu") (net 5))
 (segment (start 119.525 234.9) (end 125.22404 240.59904) (width 1) (layer "B.Cu") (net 5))
 (segment (start 119.525 193.4) (end 119.525 232.4) (width 1) (layer "B.Cu") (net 5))
 (segment (start 285.61 81.64) (end 285.61 80.71) (width 1) (layer "B.Cu") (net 5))
 (segment (start 256.209843 173.4) (end 256.209843 133.4) (width 1) (layer "B.Cu") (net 5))
 (segment (start 231.05096 240.59904) (end 256.209843 215.440157) (width 1) (layer "B.Cu") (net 5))
 (segment (start 258.749843 173.4) (end 258.749843 212.4) (width 1) (layer "B.Cu") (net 6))
 (segment (start 284.05 86) (end 288.15 81.9) (width 1) (layer "B.Cu") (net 6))
 (segment (start 116.985 232.4) (end 116.985 234.9) (width 1) (layer "B.Cu") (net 6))
 (segment (start 116.985 154.4) (end 116.985 193.4) (width 1) (layer "B.Cu") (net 6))
 (segment (start 258.749843 91.850157) (end 264.6 86) (width 1) (layer "B.Cu") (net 6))
 (segment (start 232.25144 241.89856) (end 258.749843 215.400157) (width 1) (layer "B.Cu") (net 6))
 (segment (start 264.6 86) (end 284.05 86) (width 1) (layer "B.Cu") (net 6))
 (segment (start 258.749843 95.4) (end 258.749843 133.4) (width 1) (layer "B.Cu") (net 6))
 (segment (start 288.15 81.9) (end 288.15 80.71) (width 1) (layer "B.Cu") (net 6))
 (segment (start 258.749843 95.4) (end 258.749843 91.850157) (width 1) (layer "B.Cu") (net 6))
 (segment (start 258.749843 215.400157) (end 258.749843 212.4) (width 1) (layer "B.Cu") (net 6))
 (segment (start 123.98356 241.89856) (end 232.25144 241.89856) (width 1) (layer "B.Cu") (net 6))
 (segment (start 116.985 154.4) (end 116.985 115.4) (width 1) (layer "B.Cu") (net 6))
 (segment (start 116.985 234.9) (end 123.98356 241.89856) (width 1) (layer "B.Cu") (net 6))
 (segment (start 258.749843 133.4) (end 258.749843 173.4) (width 1) (layer "B.Cu") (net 6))
 (segment (start 116.985 232.4) (end 116.985 193.4) (width 1) (layer "B.Cu") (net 6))
 (segment (start 261.289843 91.810157) (end 265.55 87.55) (width 1) (layer "B.Cu") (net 7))
 (segment (start 114.445 115.4) (end 114.445 154.4) (width 1) (layer "B.Cu") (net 7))
 (segment (start 114.445 234.9) (end 122.74308 243.19808) (width 1) (layer "B.Cu") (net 7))
 (segment (start 114.445 232.4) (end 114.445 234.9) (width 1) (layer "B.Cu") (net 7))
 (segment (start 265.55 87.55) (end 284.75 87.55) (width 1) (layer "B.Cu") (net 7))
 (segment (start 261.289843 215.510157) (end 261.289843 212.4) (width 1) (layer "B.Cu") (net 7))
 (segment (start 261.289843 95.4) (end 261.289843 91.810157) (width 1) (layer "B.Cu") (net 7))
 (segment (start 114.445 154.4) (end 114.445 193.4) (width 1) (layer "B.Cu") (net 7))
 (segment (start 261.289843 212.4) (end 261.289843 173.4) (width 1) (layer "B.Cu") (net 7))
 (segment (start 290.69 81.61) (end 290.69 80.71) (width 1) (layer "B.Cu") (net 7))
 (segment (start 114.445 193.4) (end 114.445 232.4) (width 1) (layer "B.Cu") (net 7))
 (segment (start 284.75 87.55) (end 290.69 81.61) (width 1) (layer "B.Cu") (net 7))
 (segment (start 233.60192 243.19808) (end 261.289843 215.510157) (width 1) (layer "B.Cu") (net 7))
 (segment (start 261.289843 173.4) (end 261.289843 133.4) (width 1) (layer "B.Cu") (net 7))
 (segment (start 122.74308 243.19808) (end 233.60192 243.19808) (width 1) (layer "B.Cu") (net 7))
 (segment (start 261.289843 133.4) (end 261.289843 95.4) (width 1) (layer "B.Cu") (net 7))
 (segment (start 291.15096 71.09904) (end 293.23 69.02) (width 1) (layer "F.Cu") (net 4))
 (segment (start 260.5 76.655) (end 266.282798 76.655) (width 1) (layer "F.Cu") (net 4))
 (segment (start 266.282798 76.655) (end 271.838758 71.09904) (width 1) (layer "F.Cu") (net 4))
 (segment (start 271.838758 71.09904) (end 291.15096 71.09904) (width 1) (layer "F.Cu") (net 4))
 (segment (start 293.23 69.02) (end 293.23 65.47) (width 1) (layer "F.Cu") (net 4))
 (segment (start 251.129843 212.4) (end 251.129843 173.4) (width 1) (layer "B.Cu") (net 4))
 (segment (start 124.605 115.4) (end 124.605 154.4) (width 1) (layer "B.Cu") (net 4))
 (segment (start 251.129843 215.670157) (end 251.129843 212.4) (width 1) (layer "B.Cu") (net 4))
 (segment (start 124.605 234.555) (end 128.05 238) (width 1) (layer "B.Cu") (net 4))
 (segment (start 251.129843 95.4) (end 251.129843 80.220157) (width 1) (layer "B.Cu") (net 4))
 (segment (start 228.8 238) (end 251.129843 215.670157) (width 1) (layer "B.Cu") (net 4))
 (segment (start 124.605 193.4) (end 124.605 232.4) (width 1) (layer "B.Cu") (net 4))
 (segment (start 128.05 238) (end 228.8 238) (width 1) (layer "B.Cu") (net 4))
 (segment (start 251.129843 133.4) (end 251.129843 95.4) (width 1) (layer "B.Cu") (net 4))
 (segment (start 254.695 76.655) (end 260.5 76.655) (width 1) (layer "B.Cu") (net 4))
 (segment (start 124.605 232.4) (end 124.605 234.555) (width 1) (layer "B.Cu") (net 4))
 (segment (start 251.129843 173.4) (end 251.129843 133.4) (width 1) (layer "B.Cu") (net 4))
 (segment (start 251.129843 80.220157) (end 254.695 76.655) (width 1) (layer "B.Cu") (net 4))
 (segment (start 124.605 154.4) (end 124.605 193.4) (width 1) (layer "B.Cu") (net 4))
 (segment (start 266.985 74.115) (end 271.30048 69.79952) (width 1) (layer "F.Cu") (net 3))
 (segment (start 290.69 68.76) (end 290.69 65.47) (width 1) (layer "F.Cu") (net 3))
 (segment (start 260.5 74.115) (end 266.985 74.115) (width 1) (layer "F.Cu") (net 3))
 (segment (start 271.30048 69.79952) (end 289.65048 69.79952) (width 1) (layer "F.Cu") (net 3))
 (segment (start 289.65048 69.79952) (end 290.69 68.76) (width 1) (layer "F.Cu") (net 3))
 (segment (start 127.145 193.4) (end 127.145 232.4) (width 1) (layer "B.Cu") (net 3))
 (segment (start 248.589843 212.4) (end 248.589843 173.4) (width 1) (layer "B.Cu") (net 3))
 (segment (start 127.145 234.845) (end 128.9 236.6) (width 1) (layer "B.Cu") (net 3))
 (segment (start 227.5 236.6) (end 248.589843 215.510157) (width 1) (layer "B.Cu") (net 3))
 (segment (start 248.589843 215.510157) (end 248.589843 212.4) (width 1) (layer "B.Cu") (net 3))
 (segment (start 127.145 232.4) (end 127.145 234.845) (width 1) (layer "B.Cu") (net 3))
 (segment (start 128.9 236.6) (end 227.5 236.6) (width 1) (layer "B.Cu") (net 3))
 (segment (start 260.5 74.115) (end 253.685 74.115) (width 1) (layer "B.Cu") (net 3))
 (segment (start 248.589843 133.4) (end 248.589843 95.4) (width 1) (layer "B.Cu") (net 3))
 (segment (start 248.589843 173.4) (end 248.589843 133.4) (width 1) (layer "B.Cu") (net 3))
 (segment (start 127.145 154.4) (end 127.145 193.4) (width 1) (layer "B.Cu") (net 3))
 (segment (start 248.589843 79.210157) (end 248.589843 95.4) (width 1) (layer "B.Cu") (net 3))
 (segment (start 127.145 115.4) (end 127.145 154.4) (width 1) (layer "B.Cu") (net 3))
 (segment (start 253.685 74.115) (end 248.589843 79.210157) (width 1) (layer "B.Cu") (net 3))
 (segment (start 283.07 62.47) (end 283.07 65.47) (width 1) (layer "B.Cu") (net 28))
 (segment (start 282.0625 58.1) (end 282.0625 61.4625) (width 1) (layer "B.Cu") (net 28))
 (segment (start 282.0625 61.4625) (end 283.07 62.47) (width 1) (layer "B.Cu") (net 28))
 (segment (start 246.049843 95.4) (end 246.049843 94.3) (width 1) (layer "F.Cu") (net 2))
 (segment (start 246.049843 94.3) (end 247.249843 93.1) (width 1) (layer "F.Cu") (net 2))
 (segment (start 263.829843 94.3) (end 263.829843 95.4) (width 1) (layer "F.Cu") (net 2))
 (segment (start 262.629843 93.1) (end 263.829843 94.3) (width 1) (layer "F.Cu") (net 2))
 (segment (start 247.249843 93.1) (end 262.629843 93.1) (width 1) (layer "F.Cu") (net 2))
 (segment (start 233.5 62.1) (end 236.905 65.505) (width 1) (layer "B.Cu") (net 2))
 (segment (start 121.505 244.5) (end 235 244.5) (width 1) (layer "B.Cu") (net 2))
 (segment (start 130.5 235.25) (end 226.15 235.25) (width 1) (layer "B.Cu") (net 2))
 (segment (start 240.067657 76.230157) (end 240.9375 77.1) (width 1) (layer "B.Cu") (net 2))
 (segment (start 129.685 154.4) (end 129.685 193.4) (width 1) (layer "B.Cu") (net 2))
 (segment (start 129.685 193.4) (end 129.685 232.4) (width 1) (layer "B.Cu") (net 2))
 (segment (start 233.5 57.1) (end 233.5 62.1) (width 1) (layer "B.Cu") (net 2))
 (segment (start 129.685 115.4) (end 129.685 154.4) (width 1) (layer "B.Cu") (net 2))
 (segment (start 275.45 65.47) (end 260.87 65.47) (width 1) (layer "B.Cu") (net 2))
 (segment (start 236.905 65.505) (end 240.067657 65.505) (width 1) (layer "B.Cu") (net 2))
 (segment (start 263.829843 133.4) (end 263.829843 173.4) (width 1) (layer "B.Cu") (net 2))
 (segment (start 263.829843 215.670157) (end 263.829843 212.4) (width 1) (layer "B.Cu") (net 2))
 (segment (start 246.049843 82.212343) (end 246.049843 95.4) (width 1) (layer "B.Cu") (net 2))
 (segment (start 263.829843 133.4) (end 263.829843 95.4) (width 1) (layer "B.Cu") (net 2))
 (segment (start 246.049843 215.350157) (end 246.049843 212.4) (width 1) (layer "B.Cu") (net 2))
 (segment (start 235 244.5) (end 263.829843 215.670157) (width 1) (layer "B.Cu") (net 2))
 (segment (start 260.87 65.47) (end 252.5 57.1) (width 1) (layer "B.Cu") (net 2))
 (segment (start 246.049843 95.4) (end 246.049843 133.4) (width 1) (layer "B.Cu") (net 2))
 (segment (start 240.067657 65.505) (end 240.067657 76.230157) (width 1) (layer "B.Cu") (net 2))
 (segment (start 263.829843 173.4) (end 263.829843 212.4) (width 1) (layer "B.Cu") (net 2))
 (segment (start 246.049843 212.4) (end 246.049843 173.4) (width 1) (layer "B.Cu") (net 2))
 (segment (start 246.049843 173.4) (end 246.049843 133.4) (width 1) (layer "B.Cu") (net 2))
 (segment (start 111.905 232.4) (end 111.905 234.9) (width 1) (layer "B.Cu") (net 2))
 (segment (start 226.15 235.25) (end 246.049843 215.350157) (width 1) (layer "B.Cu") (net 2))
 (segment (start 111.905 234.9) (end 121.505 244.5) (width 1) (layer "B.Cu") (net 2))
 (segment (start 240.9375 77.1) (end 246.049843 82.212343) (width 1) (layer "B.Cu") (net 2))
 (segment (start 111.905 154.4) (end 111.905 193.4) (width 1) (layer "B.Cu") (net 2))
 (segment (start 129.685 234.435) (end 130.5 235.25) (width 1) (layer "B.Cu") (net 2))
 (segment (start 252.5 57.1) (end 233.5 57.1) (width 1) (layer "B.Cu") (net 2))
 (segment (start 129.685 232.4) (end 129.685 234.435) (width 1) (layer "B.Cu") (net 2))
 (segment (start 111.905 115.4) (end 111.905 154.4) (width 1) (layer "B.Cu") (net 2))
 (segment (start 111.905 232.4) (end 111.905 193.4) (width 1) (layer "B.Cu") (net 2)))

